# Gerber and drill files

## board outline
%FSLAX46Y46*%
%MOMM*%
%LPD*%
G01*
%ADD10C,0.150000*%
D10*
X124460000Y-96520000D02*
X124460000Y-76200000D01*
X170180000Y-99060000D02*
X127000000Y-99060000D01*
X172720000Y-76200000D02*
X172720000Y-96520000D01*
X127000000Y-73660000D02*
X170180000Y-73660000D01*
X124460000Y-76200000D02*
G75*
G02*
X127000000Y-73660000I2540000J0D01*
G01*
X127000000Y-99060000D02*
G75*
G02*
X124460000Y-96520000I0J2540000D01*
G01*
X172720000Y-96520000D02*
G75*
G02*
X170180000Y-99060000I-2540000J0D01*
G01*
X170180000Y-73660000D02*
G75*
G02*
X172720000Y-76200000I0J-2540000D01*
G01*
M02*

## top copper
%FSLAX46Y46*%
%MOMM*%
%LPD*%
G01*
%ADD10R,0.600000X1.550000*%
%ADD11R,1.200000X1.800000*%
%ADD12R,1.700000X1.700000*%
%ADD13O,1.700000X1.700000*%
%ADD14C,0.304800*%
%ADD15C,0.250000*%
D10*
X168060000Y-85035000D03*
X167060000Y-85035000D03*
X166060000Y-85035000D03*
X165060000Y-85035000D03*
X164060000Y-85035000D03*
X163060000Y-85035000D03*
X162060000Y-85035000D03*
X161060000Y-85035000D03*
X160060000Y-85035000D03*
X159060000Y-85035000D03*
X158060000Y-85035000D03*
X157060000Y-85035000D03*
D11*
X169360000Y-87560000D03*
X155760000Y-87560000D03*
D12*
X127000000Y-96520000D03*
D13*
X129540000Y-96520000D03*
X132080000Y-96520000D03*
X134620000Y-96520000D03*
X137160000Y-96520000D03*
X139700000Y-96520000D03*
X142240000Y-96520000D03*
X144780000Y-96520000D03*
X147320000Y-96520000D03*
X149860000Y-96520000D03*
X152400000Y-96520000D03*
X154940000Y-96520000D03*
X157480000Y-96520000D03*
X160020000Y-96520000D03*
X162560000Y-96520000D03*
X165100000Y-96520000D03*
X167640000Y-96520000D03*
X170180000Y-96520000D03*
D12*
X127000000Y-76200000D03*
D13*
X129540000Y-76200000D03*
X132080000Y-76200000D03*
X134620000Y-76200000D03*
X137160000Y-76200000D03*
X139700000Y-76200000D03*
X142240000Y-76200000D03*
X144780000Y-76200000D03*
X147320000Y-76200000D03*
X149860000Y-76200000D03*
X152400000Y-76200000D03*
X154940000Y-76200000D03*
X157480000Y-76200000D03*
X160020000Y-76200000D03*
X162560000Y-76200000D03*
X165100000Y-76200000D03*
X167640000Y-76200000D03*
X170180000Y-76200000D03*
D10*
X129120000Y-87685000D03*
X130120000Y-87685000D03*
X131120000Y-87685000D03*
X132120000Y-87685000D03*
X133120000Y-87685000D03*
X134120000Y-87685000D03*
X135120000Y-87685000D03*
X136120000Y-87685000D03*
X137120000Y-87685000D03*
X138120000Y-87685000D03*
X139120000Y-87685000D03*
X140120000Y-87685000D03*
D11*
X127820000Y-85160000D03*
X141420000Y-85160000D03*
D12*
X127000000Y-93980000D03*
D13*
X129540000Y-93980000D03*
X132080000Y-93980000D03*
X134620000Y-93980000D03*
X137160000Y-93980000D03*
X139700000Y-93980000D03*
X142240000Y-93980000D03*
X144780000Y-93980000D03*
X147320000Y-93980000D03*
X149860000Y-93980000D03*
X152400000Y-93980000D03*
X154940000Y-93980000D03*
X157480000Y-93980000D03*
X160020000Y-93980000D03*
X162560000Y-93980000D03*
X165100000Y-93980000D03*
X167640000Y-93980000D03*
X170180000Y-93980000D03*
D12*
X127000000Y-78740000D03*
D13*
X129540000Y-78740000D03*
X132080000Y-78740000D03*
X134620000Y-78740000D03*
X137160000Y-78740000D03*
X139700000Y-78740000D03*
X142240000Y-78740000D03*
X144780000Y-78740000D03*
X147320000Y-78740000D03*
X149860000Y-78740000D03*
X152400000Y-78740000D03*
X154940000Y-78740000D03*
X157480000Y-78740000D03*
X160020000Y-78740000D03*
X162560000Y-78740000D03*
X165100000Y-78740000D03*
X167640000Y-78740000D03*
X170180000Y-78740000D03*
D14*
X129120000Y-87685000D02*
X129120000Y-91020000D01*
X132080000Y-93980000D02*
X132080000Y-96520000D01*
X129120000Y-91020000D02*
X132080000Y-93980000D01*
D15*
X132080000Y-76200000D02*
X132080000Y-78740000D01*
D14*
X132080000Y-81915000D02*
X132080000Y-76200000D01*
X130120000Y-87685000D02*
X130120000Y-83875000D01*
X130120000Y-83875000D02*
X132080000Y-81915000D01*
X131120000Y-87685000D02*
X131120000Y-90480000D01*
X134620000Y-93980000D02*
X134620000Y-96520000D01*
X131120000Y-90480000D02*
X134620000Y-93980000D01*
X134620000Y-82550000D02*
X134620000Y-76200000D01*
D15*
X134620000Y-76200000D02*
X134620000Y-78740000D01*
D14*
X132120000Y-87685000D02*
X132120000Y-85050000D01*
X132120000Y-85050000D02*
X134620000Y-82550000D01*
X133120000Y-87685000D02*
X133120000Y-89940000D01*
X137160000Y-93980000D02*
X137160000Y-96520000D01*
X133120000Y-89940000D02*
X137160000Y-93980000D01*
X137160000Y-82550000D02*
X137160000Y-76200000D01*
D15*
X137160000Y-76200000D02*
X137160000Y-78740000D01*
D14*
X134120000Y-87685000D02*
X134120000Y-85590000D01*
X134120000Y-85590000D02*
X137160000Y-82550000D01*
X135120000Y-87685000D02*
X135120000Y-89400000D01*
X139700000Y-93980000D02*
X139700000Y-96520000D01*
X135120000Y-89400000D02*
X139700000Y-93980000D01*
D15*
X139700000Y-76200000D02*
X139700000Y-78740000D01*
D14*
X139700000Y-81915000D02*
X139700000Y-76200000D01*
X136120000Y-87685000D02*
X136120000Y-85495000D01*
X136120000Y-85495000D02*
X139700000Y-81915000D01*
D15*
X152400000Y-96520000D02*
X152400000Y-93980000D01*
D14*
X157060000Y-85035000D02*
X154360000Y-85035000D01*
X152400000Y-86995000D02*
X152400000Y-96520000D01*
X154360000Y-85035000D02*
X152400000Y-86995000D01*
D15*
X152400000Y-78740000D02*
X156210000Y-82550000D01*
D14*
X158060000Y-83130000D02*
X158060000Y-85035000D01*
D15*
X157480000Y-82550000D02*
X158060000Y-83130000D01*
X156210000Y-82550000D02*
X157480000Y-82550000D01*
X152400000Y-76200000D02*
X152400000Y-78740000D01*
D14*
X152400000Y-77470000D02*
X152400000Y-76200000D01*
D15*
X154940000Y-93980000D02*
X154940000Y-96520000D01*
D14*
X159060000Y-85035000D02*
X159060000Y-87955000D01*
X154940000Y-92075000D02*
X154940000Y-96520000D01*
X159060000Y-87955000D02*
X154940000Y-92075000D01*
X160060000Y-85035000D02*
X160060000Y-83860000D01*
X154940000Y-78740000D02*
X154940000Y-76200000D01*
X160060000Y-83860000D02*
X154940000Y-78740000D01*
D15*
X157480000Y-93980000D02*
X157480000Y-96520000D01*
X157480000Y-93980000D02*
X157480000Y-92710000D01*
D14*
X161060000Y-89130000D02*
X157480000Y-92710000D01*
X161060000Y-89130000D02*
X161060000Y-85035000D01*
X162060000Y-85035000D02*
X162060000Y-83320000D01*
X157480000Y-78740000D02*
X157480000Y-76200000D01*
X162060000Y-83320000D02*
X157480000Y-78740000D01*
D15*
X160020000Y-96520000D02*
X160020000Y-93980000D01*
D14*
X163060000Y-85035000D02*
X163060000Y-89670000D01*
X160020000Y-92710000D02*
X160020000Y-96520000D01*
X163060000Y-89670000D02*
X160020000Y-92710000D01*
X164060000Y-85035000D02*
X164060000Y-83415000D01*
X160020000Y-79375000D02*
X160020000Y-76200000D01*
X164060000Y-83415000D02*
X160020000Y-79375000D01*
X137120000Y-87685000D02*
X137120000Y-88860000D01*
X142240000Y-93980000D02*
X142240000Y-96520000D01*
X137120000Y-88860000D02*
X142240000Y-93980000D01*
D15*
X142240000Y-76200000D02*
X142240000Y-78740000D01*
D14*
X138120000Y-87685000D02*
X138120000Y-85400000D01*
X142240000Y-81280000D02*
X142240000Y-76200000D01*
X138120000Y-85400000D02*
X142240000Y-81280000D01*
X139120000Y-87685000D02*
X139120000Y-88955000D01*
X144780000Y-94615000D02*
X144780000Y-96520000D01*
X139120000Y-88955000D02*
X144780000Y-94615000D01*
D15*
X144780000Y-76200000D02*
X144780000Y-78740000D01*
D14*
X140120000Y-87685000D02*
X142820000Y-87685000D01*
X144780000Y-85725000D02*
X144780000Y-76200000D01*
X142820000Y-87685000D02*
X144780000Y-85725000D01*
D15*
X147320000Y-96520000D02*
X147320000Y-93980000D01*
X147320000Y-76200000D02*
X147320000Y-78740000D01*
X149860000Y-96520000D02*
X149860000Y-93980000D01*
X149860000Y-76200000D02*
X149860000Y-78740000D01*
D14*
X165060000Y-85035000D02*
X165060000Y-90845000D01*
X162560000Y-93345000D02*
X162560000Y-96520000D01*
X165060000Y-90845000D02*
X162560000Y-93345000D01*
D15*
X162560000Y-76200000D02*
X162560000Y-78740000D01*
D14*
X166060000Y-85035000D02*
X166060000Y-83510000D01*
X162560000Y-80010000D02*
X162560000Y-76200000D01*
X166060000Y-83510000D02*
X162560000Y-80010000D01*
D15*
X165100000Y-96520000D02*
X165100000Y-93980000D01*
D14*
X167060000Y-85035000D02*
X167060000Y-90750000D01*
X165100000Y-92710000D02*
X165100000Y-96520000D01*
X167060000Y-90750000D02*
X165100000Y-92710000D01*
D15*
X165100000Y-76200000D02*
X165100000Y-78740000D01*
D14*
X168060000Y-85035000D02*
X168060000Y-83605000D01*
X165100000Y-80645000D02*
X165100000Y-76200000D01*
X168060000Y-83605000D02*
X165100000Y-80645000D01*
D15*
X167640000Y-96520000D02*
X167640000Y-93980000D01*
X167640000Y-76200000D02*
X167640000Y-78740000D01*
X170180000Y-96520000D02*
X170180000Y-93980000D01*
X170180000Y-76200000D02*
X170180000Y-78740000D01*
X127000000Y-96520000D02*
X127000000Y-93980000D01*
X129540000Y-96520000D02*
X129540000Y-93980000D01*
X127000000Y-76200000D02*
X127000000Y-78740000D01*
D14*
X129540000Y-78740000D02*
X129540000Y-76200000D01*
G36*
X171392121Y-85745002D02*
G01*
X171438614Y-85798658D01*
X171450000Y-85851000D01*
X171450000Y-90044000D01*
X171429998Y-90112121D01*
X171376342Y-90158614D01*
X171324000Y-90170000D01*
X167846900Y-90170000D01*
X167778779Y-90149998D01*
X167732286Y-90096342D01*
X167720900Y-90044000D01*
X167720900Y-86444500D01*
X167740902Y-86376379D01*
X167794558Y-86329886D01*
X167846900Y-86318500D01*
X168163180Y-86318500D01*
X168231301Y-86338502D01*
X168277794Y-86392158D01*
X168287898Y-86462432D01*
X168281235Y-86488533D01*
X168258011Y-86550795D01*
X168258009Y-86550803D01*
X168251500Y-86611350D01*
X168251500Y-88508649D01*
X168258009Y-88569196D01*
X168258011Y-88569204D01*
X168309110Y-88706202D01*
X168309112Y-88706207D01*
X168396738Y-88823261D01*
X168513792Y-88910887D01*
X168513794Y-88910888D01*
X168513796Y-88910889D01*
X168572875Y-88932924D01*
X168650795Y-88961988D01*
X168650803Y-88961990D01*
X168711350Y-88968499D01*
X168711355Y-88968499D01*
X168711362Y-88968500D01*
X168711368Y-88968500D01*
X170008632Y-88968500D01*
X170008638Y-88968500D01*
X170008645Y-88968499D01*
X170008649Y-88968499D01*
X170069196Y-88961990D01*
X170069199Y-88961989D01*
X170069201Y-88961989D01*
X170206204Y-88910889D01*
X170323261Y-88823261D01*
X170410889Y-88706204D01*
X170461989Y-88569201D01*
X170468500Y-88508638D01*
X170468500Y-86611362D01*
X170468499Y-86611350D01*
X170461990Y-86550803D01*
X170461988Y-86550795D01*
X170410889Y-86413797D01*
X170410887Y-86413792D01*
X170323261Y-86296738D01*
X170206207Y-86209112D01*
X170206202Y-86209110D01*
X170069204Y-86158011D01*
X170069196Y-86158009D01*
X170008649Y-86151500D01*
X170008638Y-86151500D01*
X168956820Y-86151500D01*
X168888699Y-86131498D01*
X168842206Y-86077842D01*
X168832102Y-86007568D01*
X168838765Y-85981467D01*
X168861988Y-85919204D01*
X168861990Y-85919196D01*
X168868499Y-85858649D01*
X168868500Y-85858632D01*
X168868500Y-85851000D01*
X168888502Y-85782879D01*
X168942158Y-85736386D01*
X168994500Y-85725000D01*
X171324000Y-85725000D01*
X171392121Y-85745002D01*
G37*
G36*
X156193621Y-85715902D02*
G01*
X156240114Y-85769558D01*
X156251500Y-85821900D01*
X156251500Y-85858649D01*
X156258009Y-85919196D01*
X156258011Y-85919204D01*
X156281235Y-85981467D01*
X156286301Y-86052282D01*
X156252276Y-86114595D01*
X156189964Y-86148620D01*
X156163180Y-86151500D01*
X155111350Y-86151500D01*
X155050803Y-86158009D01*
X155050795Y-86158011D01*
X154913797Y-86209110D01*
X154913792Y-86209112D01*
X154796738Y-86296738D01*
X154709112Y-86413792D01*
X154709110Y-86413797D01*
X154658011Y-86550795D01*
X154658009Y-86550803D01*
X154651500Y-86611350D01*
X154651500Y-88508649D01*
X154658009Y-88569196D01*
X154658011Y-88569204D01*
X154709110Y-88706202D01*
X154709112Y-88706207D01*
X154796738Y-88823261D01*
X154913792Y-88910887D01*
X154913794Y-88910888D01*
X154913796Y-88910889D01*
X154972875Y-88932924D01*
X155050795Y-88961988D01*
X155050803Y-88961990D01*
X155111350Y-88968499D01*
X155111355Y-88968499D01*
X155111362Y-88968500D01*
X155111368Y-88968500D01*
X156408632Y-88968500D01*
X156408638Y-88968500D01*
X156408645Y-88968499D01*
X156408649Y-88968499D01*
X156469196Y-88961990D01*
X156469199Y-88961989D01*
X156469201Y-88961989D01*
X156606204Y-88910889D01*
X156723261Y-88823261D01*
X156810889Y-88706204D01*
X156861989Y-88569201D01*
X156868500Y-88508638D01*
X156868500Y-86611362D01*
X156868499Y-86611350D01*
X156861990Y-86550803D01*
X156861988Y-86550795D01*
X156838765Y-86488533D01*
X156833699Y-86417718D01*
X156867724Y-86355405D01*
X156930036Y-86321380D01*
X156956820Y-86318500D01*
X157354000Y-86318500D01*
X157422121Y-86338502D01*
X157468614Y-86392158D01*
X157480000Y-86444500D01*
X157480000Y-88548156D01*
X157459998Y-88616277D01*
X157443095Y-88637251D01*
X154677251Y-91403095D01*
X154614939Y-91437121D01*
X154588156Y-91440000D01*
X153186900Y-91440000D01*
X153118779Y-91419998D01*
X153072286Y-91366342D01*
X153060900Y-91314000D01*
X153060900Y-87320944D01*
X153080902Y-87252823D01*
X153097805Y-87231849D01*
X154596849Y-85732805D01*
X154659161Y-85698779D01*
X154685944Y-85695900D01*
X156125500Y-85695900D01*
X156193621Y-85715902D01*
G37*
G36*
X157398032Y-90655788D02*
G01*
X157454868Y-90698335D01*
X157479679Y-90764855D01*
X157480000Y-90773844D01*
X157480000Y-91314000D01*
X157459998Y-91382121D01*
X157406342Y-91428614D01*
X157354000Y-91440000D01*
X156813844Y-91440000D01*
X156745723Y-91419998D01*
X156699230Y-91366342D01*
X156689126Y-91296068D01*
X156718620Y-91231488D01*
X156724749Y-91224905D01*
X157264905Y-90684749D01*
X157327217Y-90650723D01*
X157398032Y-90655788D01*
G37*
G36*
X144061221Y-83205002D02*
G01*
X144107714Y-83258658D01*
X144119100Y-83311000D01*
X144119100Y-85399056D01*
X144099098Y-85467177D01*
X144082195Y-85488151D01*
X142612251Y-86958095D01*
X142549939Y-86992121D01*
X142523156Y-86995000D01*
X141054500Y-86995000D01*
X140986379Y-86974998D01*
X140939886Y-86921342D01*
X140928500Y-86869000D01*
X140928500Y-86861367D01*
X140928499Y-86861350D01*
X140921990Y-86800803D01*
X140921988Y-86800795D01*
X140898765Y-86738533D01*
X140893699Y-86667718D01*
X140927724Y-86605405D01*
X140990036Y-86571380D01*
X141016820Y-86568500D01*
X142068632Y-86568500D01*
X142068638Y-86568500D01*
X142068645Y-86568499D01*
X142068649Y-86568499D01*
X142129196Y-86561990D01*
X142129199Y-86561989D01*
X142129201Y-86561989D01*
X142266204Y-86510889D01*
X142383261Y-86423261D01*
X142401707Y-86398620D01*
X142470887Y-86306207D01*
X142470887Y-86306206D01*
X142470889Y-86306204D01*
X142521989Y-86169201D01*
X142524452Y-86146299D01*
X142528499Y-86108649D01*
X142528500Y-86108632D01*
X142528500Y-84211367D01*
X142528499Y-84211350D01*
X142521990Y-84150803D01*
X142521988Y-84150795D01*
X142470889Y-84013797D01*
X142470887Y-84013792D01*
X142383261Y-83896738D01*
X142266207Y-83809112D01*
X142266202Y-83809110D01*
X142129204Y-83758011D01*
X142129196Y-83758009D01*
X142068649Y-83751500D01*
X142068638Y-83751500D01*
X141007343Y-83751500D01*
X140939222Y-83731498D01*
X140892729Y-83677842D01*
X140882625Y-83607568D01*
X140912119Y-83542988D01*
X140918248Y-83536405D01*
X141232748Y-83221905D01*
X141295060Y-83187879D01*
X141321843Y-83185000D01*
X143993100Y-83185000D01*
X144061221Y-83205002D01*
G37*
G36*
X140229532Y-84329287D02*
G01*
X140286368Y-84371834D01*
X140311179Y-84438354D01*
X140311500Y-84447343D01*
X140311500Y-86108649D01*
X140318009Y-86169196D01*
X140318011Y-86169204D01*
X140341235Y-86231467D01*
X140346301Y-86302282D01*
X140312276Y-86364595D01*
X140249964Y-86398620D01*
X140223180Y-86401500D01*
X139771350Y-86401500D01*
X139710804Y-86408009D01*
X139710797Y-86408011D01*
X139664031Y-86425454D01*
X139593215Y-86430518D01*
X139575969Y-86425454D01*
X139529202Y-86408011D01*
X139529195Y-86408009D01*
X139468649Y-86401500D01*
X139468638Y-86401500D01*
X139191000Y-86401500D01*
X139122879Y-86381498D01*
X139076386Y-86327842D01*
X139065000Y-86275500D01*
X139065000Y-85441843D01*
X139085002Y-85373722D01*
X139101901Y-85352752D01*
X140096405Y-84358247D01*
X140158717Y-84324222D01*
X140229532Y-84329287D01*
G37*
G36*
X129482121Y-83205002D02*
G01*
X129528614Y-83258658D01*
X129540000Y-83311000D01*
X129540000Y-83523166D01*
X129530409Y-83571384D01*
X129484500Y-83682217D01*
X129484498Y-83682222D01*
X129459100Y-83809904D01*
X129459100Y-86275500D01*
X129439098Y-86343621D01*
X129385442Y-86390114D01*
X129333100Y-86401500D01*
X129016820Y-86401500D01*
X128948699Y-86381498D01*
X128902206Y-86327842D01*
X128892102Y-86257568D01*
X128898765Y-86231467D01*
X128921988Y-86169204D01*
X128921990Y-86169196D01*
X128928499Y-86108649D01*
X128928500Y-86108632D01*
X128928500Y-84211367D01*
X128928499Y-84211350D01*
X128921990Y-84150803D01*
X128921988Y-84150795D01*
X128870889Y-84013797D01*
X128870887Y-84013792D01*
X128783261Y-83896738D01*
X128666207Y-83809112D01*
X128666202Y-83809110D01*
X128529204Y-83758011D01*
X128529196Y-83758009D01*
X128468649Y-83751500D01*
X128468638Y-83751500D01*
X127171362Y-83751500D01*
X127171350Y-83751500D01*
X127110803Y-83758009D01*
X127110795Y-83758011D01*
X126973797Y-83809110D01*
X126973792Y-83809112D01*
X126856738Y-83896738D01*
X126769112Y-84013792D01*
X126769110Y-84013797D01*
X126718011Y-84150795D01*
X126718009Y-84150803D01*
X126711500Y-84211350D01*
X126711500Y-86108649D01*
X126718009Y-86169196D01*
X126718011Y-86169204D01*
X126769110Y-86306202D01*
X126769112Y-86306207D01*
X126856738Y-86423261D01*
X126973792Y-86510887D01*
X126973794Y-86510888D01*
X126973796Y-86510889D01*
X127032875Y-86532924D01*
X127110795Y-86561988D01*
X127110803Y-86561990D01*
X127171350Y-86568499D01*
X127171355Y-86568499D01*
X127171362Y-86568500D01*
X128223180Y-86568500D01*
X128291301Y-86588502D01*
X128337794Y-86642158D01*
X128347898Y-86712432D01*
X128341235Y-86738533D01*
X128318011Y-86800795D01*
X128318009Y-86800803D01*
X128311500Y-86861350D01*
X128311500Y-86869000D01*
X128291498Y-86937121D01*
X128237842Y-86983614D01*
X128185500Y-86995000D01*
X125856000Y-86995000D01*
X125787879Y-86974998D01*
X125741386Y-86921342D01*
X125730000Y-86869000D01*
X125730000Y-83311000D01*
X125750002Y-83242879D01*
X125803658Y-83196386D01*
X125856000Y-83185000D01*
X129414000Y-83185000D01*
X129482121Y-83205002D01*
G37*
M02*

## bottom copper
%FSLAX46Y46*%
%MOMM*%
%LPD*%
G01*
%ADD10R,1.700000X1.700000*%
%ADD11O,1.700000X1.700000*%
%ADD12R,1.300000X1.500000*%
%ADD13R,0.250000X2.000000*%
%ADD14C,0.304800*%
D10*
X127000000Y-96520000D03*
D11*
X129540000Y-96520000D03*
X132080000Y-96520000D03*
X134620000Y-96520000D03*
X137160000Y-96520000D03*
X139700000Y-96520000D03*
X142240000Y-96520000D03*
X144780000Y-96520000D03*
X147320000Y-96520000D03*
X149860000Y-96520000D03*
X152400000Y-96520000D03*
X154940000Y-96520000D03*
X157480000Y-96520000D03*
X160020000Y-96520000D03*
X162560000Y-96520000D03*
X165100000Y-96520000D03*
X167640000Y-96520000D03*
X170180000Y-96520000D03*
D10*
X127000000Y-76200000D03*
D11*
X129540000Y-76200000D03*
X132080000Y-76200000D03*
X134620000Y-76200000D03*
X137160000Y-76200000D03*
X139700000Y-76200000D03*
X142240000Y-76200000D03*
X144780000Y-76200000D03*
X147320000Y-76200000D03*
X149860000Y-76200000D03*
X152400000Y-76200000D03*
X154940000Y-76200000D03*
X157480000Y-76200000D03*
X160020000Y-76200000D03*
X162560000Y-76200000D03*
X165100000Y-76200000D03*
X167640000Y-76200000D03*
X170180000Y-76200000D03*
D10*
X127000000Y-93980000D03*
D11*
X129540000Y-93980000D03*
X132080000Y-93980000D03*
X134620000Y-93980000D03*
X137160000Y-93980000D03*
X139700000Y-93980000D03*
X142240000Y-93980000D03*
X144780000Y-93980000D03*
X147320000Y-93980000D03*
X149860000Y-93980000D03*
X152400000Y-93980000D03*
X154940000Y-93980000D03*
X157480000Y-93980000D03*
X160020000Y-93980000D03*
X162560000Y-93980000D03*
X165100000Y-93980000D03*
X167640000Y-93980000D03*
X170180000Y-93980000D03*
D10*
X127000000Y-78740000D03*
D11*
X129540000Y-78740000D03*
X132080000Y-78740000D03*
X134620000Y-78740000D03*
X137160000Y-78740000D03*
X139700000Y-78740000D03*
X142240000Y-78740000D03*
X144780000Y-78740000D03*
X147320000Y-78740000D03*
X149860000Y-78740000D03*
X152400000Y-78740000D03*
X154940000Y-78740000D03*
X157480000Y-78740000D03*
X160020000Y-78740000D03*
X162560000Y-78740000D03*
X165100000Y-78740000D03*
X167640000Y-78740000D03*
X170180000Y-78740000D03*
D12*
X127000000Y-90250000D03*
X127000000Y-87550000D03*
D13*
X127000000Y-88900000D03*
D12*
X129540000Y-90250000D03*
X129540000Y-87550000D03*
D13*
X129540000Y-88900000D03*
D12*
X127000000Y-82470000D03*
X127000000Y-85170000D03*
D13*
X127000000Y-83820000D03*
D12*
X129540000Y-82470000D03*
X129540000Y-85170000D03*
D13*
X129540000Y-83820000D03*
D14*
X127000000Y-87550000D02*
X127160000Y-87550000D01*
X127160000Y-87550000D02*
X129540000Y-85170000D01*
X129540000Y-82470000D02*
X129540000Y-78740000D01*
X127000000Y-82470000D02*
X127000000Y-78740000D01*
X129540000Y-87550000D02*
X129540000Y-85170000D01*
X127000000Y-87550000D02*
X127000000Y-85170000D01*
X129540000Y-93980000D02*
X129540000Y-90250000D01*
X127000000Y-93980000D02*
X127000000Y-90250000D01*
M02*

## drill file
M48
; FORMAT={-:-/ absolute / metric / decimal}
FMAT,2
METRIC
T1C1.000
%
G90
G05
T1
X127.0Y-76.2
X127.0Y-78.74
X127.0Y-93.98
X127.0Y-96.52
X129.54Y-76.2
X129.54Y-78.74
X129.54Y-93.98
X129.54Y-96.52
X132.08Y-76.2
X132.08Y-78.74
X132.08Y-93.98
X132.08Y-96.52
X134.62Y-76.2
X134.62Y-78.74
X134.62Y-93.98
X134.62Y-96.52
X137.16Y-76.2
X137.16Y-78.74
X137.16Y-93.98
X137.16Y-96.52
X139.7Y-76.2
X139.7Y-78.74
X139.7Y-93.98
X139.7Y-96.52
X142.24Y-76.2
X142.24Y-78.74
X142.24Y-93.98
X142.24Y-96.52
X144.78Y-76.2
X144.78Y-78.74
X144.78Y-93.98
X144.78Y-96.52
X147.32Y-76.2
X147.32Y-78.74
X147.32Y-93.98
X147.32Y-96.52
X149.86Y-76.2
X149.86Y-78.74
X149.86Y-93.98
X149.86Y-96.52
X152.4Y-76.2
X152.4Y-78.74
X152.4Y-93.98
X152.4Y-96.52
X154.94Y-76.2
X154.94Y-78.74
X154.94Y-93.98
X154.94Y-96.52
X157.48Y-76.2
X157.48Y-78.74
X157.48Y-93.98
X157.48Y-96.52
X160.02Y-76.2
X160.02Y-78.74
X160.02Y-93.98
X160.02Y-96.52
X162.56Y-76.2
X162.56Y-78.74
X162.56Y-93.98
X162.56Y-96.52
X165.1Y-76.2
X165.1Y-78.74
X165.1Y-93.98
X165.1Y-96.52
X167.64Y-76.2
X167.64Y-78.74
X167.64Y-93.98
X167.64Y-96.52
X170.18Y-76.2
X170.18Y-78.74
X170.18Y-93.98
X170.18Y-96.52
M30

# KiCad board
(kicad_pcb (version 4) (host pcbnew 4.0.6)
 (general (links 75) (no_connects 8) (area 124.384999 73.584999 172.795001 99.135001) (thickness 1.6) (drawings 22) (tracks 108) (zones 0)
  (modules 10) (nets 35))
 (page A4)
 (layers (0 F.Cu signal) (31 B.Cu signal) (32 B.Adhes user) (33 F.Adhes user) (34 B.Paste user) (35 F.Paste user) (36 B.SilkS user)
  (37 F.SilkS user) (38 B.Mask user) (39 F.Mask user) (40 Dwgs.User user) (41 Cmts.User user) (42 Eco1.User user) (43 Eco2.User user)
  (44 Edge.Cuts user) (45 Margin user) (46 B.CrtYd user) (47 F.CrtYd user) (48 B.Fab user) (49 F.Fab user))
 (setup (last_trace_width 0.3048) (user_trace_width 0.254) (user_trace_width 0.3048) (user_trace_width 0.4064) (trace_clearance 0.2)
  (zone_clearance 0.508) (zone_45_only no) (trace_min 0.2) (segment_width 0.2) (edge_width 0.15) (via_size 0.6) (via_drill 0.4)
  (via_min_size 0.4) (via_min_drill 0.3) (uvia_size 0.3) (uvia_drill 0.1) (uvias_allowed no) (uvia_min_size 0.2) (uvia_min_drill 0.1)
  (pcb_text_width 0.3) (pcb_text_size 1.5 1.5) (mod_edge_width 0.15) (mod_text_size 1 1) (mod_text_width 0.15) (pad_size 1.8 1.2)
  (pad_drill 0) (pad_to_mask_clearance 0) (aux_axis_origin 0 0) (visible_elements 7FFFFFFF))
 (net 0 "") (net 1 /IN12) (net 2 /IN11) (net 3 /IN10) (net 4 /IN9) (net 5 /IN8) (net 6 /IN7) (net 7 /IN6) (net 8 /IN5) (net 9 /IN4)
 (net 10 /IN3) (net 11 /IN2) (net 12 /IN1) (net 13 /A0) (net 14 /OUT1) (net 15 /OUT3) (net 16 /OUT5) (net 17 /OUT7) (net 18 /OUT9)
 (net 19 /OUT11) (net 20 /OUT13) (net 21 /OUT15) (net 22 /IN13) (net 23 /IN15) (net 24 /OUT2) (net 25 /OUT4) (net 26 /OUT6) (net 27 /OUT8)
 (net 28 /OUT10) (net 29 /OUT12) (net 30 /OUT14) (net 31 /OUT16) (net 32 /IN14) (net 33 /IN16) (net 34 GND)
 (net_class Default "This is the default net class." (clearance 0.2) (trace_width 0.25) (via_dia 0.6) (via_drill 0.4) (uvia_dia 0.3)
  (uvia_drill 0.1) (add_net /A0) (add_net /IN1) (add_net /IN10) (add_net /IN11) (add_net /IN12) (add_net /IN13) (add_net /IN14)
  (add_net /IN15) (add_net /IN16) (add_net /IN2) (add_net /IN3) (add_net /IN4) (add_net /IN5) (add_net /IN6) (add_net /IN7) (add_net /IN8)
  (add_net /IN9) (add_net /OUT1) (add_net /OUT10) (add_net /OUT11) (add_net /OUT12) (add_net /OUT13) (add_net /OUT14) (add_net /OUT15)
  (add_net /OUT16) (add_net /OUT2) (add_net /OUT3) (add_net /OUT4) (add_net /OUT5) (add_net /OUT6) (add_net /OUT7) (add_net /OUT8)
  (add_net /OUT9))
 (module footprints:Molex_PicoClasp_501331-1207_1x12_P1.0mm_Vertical (layer F.Cu) (at 162.56 86.36 270)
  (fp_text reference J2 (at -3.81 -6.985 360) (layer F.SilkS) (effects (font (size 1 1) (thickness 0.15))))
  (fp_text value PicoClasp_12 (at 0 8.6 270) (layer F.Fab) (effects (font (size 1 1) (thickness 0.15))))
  (pad 1 smd rect (at -1.325 -5.5 270) (size 1.55 0.6) (layers F.Cu F.Paste F.Mask) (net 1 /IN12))
  (pad 2 smd rect (at -1.325 -4.5 270) (size 1.55 0.6) (layers F.Cu F.Paste F.Mask) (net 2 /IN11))
  (pad 3 smd rect (at -1.325 -3.5 270) (size 1.55 0.6) (layers F.Cu F.Paste F.Mask) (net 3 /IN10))
  (pad 4 smd rect (at -1.325 -2.5 270) (size 1.55 0.6) (layers F.Cu F.Paste F.Mask) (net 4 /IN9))
  (pad 5 smd rect (at -1.325 -1.5 270) (size 1.55 0.6) (layers F.Cu F.Paste F.Mask) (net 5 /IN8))
  (pad 6 smd rect (at -1.325 -0.5 270) (size 1.55 0.6) (layers F.Cu F.Paste F.Mask) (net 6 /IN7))
  (pad 7 smd rect (at -1.325 0.5 270) (size 1.55 0.6) (layers F.Cu F.Paste F.Mask) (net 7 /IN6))
  (pad 8 smd rect (at -1.325 1.5 270) (size 1.55 0.6) (layers F.Cu F.Paste F.Mask) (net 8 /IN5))
  (pad 9 smd rect (at -1.325 2.5 270) (size 1.55 0.6) (layers F.Cu F.Paste F.Mask) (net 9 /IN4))
  (pad 10 smd rect (at -1.325 3.5 270) (size 1.55 0.6) (layers F.Cu F.Paste F.Mask) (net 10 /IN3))
  (pad 11 smd rect (at -1.325 4.5 270) (size 1.55 0.6) (layers F.Cu F.Paste F.Mask) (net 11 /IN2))
  (pad 12 smd rect (at -1.325 5.5 270) (size 1.55 0.6) (layers F.Cu F.Paste F.Mask) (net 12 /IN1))
  (pad 13 smd rect (at 1.2 -6.8 270) (size 1.8 1.2) (layers F.Cu F.Paste F.Mask))
  (pad 13 smd rect (at 1.2 6.8 270) (size 1.8 1.2) (layers F.Cu F.Paste F.Mask)))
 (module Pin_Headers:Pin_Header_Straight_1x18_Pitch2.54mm (layer F.Cu) (at 127 96.52 90)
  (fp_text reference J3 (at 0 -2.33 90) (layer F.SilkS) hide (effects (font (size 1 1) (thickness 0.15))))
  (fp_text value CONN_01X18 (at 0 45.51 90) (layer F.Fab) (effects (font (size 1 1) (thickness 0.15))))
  (pad 1 thru_hole rect (at 0 0 90) (size 1.7 1.7) (drill 1) (layers *.Cu *.Mask) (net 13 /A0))
  (pad 2 thru_hole oval (at 0 2.54 90) (size 1.7 1.7) (drill 1) (layers *.Cu *.Mask) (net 13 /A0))
  (pad 3 thru_hole oval (at 0 5.08 90) (size 1.7 1.7) (drill 1) (layers *.Cu *.Mask) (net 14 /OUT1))
  (pad 4 thru_hole oval (at 0 7.62 90) (size 1.7 1.7) (drill 1) (layers *.Cu *.Mask) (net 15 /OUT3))
  (pad 5 thru_hole oval (at 0 10.16 90) (size 1.7 1.7) (drill 1) (layers *.Cu *.Mask) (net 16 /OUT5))
  (pad 6 thru_hole oval (at 0 12.7 90) (size 1.7 1.7) (drill 1) (layers *.Cu *.Mask) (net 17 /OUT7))
  (pad 7 thru_hole oval (at 0 15.24 90) (size 1.7 1.7) (drill 1) (layers *.Cu *.Mask) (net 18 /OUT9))
  (pad 8 thru_hole oval (at 0 17.78 90) (size 1.7 1.7) (drill 1) (layers *.Cu *.Mask) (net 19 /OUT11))
  (pad 9 thru_hole oval (at 0 20.32 90) (size 1.7 1.7) (drill 1) (layers *.Cu *.Mask) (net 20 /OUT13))
  (pad 10 thru_hole oval (at 0 22.86 90) (size 1.7 1.7) (drill 1) (layers *.Cu *.Mask) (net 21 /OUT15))
  (pad 11 thru_hole oval (at 0 25.4 90) (size 1.7 1.7) (drill 1) (layers *.Cu *.Mask) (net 12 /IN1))
  (pad 12 thru_hole oval (at 0 27.94 90) (size 1.7 1.7) (drill 1) (layers *.Cu *.Mask) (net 10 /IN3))
  (pad 13 thru_hole oval (at 0 30.48 90) (size 1.7 1.7) (drill 1) (layers *.Cu *.Mask) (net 8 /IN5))
  (pad 14 thru_hole oval (at 0 33.02 90) (size 1.7 1.7) (drill 1) (layers *.Cu *.Mask) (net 6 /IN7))
  (pad 15 thru_hole oval (at 0 35.56 90) (size 1.7 1.7) (drill 1) (layers *.Cu *.Mask) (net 4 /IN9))
  (pad 16 thru_hole oval (at 0 38.1 90) (size 1.7 1.7) (drill 1) (layers *.Cu *.Mask) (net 2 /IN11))
  (pad 17 thru_hole oval (at 0 40.64 90) (size 1.7 1.7) (drill 1) (layers *.Cu *.Mask) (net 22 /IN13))
  (pad 18 thru_hole oval (at 0 43.18 90) (size 1.7 1.7) (drill 1) (layers *.Cu *.Mask) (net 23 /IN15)))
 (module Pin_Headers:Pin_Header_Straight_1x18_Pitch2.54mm (layer F.Cu) (at 127 76.2 90)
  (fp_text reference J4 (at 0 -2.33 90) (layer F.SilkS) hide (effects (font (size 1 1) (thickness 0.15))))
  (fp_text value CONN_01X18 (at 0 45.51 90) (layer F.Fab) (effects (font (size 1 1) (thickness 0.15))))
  (pad 1 thru_hole rect (at 0 0 90) (size 1.7 1.7) (drill 1) (layers *.Cu *.Mask) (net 13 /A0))
  (pad 2 thru_hole oval (at 0 2.54 90) (size 1.7 1.7) (drill 1) (layers *.Cu *.Mask) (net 13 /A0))
  (pad 3 thru_hole oval (at 0 5.08 90) (size 1.7 1.7) (drill 1) (layers *.Cu *.Mask) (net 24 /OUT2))
  (pad 4 thru_hole oval (at 0 7.62 90) (size 1.7 1.7) (drill 1) (layers *.Cu *.Mask) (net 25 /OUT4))
  (pad 5 thru_hole oval (at 0 10.16 90) (size 1.7 1.7) (drill 1) (layers *.Cu *.Mask) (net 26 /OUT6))
  (pad 6 thru_hole oval (at 0 12.7 90) (size 1.7 1.7) (drill 1) (layers *.Cu *.Mask) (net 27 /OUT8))
  (pad 7 thru_hole oval (at 0 15.24 90) (size 1.7 1.7) (drill 1) (layers *.Cu *.Mask) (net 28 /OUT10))
  (pad 8 thru_hole oval (at 0 17.78 90) (size 1.7 1.7) (drill 1) (layers *.Cu *.Mask) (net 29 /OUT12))
  (pad 9 thru_hole oval (at 0 20.32 90) (size 1.7 1.7) (drill 1) (layers *.Cu *.Mask) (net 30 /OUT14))
  (pad 10 thru_hole oval (at 0 22.86 90) (size 1.7 1.7) (drill 1) (layers *.Cu *.Mask) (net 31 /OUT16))
  (pad 11 thru_hole oval (at 0 25.4 90) (size 1.7 1.7) (drill 1) (layers *.Cu *.Mask) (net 11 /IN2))
  (pad 12 thru_hole oval (at 0 27.94 90) (size 1.7 1.7) (drill 1) (layers *.Cu *.Mask) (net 9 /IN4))
  (pad 13 thru_hole oval (at 0 30.48 90) (size 1.7 1.7) (drill 1) (layers *.Cu *.Mask) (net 7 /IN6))
  (pad 14 thru_hole oval (at 0 33.02 90) (size 1.7 1.7) (drill 1) (layers *.Cu *.Mask) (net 5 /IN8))
  (pad 15 thru_hole oval (at 0 35.56 90) (size 1.7 1.7) (drill 1) (layers *.Cu *.Mask) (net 3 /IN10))
  (pad 16 thru_hole oval (at 0 38.1 90) (size 1.7 1.7) (drill 1) (layers *.Cu *.Mask) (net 1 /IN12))
  (pad 17 thru_hole oval (at 0 40.64 90) (size 1.7 1.7) (drill 1) (layers *.Cu *.Mask) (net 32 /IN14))
  (pad 18 thru_hole oval (at 0 43.18 90) (size 1.7 1.7) (drill 1) (layers *.Cu *.Mask) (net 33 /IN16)))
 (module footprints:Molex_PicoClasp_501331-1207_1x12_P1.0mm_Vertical (layer F.Cu) (at 134.62 86.36 90)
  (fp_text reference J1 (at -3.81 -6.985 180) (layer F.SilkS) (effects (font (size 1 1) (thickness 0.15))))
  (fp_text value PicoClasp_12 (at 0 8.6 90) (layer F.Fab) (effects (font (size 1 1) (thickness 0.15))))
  (pad 1 smd rect (at -1.325 -5.5 90) (size 1.55 0.6) (layers F.Cu F.Paste F.Mask) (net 14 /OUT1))
  (pad 2 smd rect (at -1.325 -4.5 90) (size 1.55 0.6) (layers F.Cu F.Paste F.Mask) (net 24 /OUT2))
  (pad 3 smd rect (at -1.325 -3.5 90) (size 1.55 0.6) (layers F.Cu F.Paste F.Mask) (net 15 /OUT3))
  (pad 4 smd rect (at -1.325 -2.5 90) (size 1.55 0.6) (layers F.Cu F.Paste F.Mask) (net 25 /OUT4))
  (pad 5 smd rect (at -1.325 -1.5 90) (size 1.55 0.6) (layers F.Cu F.Paste F.Mask) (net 16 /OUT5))
  (pad 6 smd rect (at -1.325 -0.5 90) (size 1.55 0.6) (layers F.Cu F.Paste F.Mask) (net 26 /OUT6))
  (pad 7 smd rect (at -1.325 0.5 90) (size 1.55 0.6) (layers F.Cu F.Paste F.Mask) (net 17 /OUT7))
  (pad 8 smd rect (at -1.325 1.5 90) (size 1.55 0.6) (layers F.Cu F.Paste F.Mask) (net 27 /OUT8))
  (pad 9 smd rect (at -1.325 2.5 90) (size 1.55 0.6) (layers F.Cu F.Paste F.Mask) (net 18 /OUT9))
  (pad 10 smd rect (at -1.325 3.5 90) (size 1.55 0.6) (layers F.Cu F.Paste F.Mask) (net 28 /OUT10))
  (pad 11 smd rect (at -1.325 4.5 90) (size 1.55 0.6) (layers F.Cu F.Paste F.Mask) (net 19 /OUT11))
  (pad 12 smd rect (at -1.325 5.5 90) (size 1.55 0.6) (layers F.Cu F.Paste F.Mask) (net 29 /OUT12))
  (pad 13 smd rect (at 1.2 -6.8 90) (size 1.8 1.2) (layers F.Cu F.Paste F.Mask))
  (pad 13 smd rect (at 1.2 6.8 90) (size 1.8 1.2) (layers F.Cu F.Paste F.Mask)))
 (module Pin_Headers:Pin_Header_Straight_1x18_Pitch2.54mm (layer F.Cu) (at 127 93.98 90)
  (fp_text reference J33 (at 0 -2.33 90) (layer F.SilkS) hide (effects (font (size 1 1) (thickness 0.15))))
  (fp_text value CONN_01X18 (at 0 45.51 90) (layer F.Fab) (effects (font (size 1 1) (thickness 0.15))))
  (pad 1 thru_hole rect (at 0 0 90) (size 1.7 1.7) (drill 1) (layers *.Cu *.Mask) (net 13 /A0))
  (pad 2 thru_hole oval (at 0 2.54 90) (size 1.7 1.7) (drill 1) (layers *.Cu *.Mask) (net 13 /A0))
  (pad 3 thru_hole oval (at 0 5.08 90) (size 1.7 1.7) (drill 1) (layers *.Cu *.Mask) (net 14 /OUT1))
  (pad 4 thru_hole oval (at 0 7.62 90) (size 1.7 1.7) (drill 1) (layers *.Cu *.Mask) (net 15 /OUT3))
  (pad 5 thru_hole oval (at 0 10.16 90) (size 1.7 1.7) (drill 1) (layers *.Cu *.Mask) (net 16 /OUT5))
  (pad 6 thru_hole oval (at 0 12.7 90) (size 1.7 1.7) (drill 1) (layers *.Cu *.Mask) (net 17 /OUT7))
  (pad 7 thru_hole oval (at 0 15.24 90) (size 1.7 1.7) (drill 1) (layers *.Cu *.Mask) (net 18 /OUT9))
  (pad 8 thru_hole oval (at 0 17.78 90) (size 1.7 1.7) (drill 1) (layers *.Cu *.Mask) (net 19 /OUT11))
  (pad 9 thru_hole oval (at 0 20.32 90) (size 1.7 1.7) (drill 1) (layers *.Cu *.Mask) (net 20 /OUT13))
  (pad 10 thru_hole oval (at 0 22.86 90) (size 1.7 1.7) (drill 1) (layers *.Cu *.Mask) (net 21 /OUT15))
  (pad 11 thru_hole oval (at 0 25.4 90) (size 1.7 1.7) (drill 1) (layers *.Cu *.Mask) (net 12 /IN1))
  (pad 12 thru_hole oval (at 0 27.94 90) (size 1.7 1.7) (drill 1) (layers *.Cu *.Mask) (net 10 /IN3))
  (pad 13 thru_hole oval (at 0 30.48 90) (size 1.7 1.7) (drill 1) (layers *.Cu *.Mask) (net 8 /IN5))
  (pad 14 thru_hole oval (at 0 33.02 90) (size 1.7 1.7) (drill 1) (layers *.Cu *.Mask) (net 6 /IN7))
  (pad 15 thru_hole oval (at 0 35.56 90) (size 1.7 1.7) (drill 1) (layers *.Cu *.Mask) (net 4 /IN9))
  (pad 16 thru_hole oval (at 0 38.1 90) (size 1.7 1.7) (drill 1) (layers *.Cu *.Mask) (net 2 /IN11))
  (pad 17 thru_hole oval (at 0 40.64 90) (size 1.7 1.7) (drill 1) (layers *.Cu *.Mask) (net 22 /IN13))
  (pad 18 thru_hole oval (at 0 43.18 90) (size 1.7 1.7) (drill 1) (layers *.Cu *.Mask) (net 23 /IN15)))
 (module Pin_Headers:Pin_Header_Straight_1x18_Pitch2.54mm (layer F.Cu) (at 127 78.74 90)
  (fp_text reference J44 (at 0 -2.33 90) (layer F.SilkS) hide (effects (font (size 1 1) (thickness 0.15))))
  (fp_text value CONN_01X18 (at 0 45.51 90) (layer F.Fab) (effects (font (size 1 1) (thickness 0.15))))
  (pad 1 thru_hole rect (at 0 0 90) (size 1.7 1.7) (drill 1) (layers *.Cu *.Mask) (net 13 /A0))
  (pad 2 thru_hole oval (at 0 2.54 90) (size 1.7 1.7) (drill 1) (layers *.Cu *.Mask) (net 13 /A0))
  (pad 3 thru_hole oval (at 0 5.08 90) (size 1.7 1.7) (drill 1) (layers *.Cu *.Mask) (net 24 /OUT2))
  (pad 4 thru_hole oval (at 0 7.62 90) (size 1.7 1.7) (drill 1) (layers *.Cu *.Mask) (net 25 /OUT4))
  (pad 5 thru_hole oval (at 0 10.16 90) (size 1.7 1.7) (drill 1) (layers *.Cu *.Mask) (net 26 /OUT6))
  (pad 6 thru_hole oval (at 0 12.7 90) (size 1.7 1.7) (drill 1) (layers *.Cu *.Mask) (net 27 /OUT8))
  (pad 7 thru_hole oval (at 0 15.24 90) (size 1.7 1.7) (drill 1) (layers *.Cu *.Mask) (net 28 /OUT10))
  (pad 8 thru_hole oval (at 0 17.78 90) (size 1.7 1.7) (drill 1) (layers *.Cu *.Mask) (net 29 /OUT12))
  (pad 9 thru_hole oval (at 0 20.32 90) (size 1.7 1.7) (drill 1) (layers *.Cu *.Mask) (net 30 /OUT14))
  (pad 10 thru_hole oval (at 0 22.86 90) (size 1.7 1.7) (drill 1) (layers *.Cu *.Mask) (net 31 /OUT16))
  (pad 11 thru_hole oval (at 0 25.4 90) (size 1.7 1.7) (drill 1) (layers *.Cu *.Mask) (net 11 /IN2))
  (pad 12 thru_hole oval (at 0 27.94 90) (size 1.7 1.7) (drill 1) (layers *.Cu *.Mask) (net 9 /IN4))
  (pad 13 thru_hole oval (at 0 30.48 90) (size 1.7 1.7) (drill 1) (layers *.Cu *.Mask) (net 7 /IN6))
  (pad 14 thru_hole oval (at 0 33.02 90) (size 1.7 1.7) (drill 1) (layers *.Cu *.Mask) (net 5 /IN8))
  (pad 15 thru_hole oval (at 0 35.56 90) (size 1.7 1.7) (drill 1) (layers *.Cu *.Mask) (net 3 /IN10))
  (pad 16 thru_hole oval (at 0 38.1 90) (size 1.7 1.7) (drill 1) (layers *.Cu *.Mask) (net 1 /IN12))
  (pad 17 thru_hole oval (at 0 40.64 90) (size 1.7 1.7) (drill 1) (layers *.Cu *.Mask) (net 32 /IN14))
  (pad 18 thru_hole oval (at 0 43.18 90) (size 1.7 1.7) (drill 1) (layers *.Cu *.Mask) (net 33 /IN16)))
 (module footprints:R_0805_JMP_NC (layer B.Cu) (at 127 88.9 90)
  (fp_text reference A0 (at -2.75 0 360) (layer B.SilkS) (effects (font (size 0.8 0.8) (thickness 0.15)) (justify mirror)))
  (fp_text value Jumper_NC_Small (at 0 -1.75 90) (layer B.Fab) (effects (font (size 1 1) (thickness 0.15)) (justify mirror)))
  (pad 1 smd rect (at -1.35 0 90) (size 1.5 1.3) (layers B.Cu B.Paste B.Mask) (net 13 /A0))
  (pad 2 smd rect (at 1.35 0 90) (size 1.5 1.3) (layers B.Cu B.Paste B.Mask) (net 13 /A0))
  (pad 1 smd rect (at 0 0 90) (size 2 0.25) (layers B.Cu B.Paste B.Mask) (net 13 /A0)))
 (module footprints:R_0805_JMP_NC (layer B.Cu) (at 129.54 88.9 90)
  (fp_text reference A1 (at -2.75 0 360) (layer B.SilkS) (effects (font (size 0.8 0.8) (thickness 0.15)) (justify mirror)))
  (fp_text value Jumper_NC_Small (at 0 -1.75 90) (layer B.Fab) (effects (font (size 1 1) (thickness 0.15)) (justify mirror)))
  (pad 1 smd rect (at -1.35 0 90) (size 1.5 1.3) (layers B.Cu B.Paste B.Mask) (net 13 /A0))
  (pad 2 smd rect (at 1.35 0 90) (size 1.5 1.3) (layers B.Cu B.Paste B.Mask) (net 13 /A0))
  (pad 1 smd rect (at 0 0 90) (size 2 0.25) (layers B.Cu B.Paste B.Mask) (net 13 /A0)))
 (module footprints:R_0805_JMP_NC (layer B.Cu) (at 127 83.82 270)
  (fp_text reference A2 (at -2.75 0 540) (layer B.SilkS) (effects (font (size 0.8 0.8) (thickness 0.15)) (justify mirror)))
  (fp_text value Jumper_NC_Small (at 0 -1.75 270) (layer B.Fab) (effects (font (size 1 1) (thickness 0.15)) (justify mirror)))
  (pad 1 smd rect (at -1.35 0 270) (size 1.5 1.3) (layers B.Cu B.Paste B.Mask) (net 13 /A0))
  (pad 2 smd rect (at 1.35 0 270) (size 1.5 1.3) (layers B.Cu B.Paste B.Mask) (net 13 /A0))
  (pad 1 smd rect (at 0 0 270) (size 2 0.25) (layers B.Cu B.Paste B.Mask) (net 13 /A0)))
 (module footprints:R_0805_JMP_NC (layer B.Cu) (at 129.54 83.82 270)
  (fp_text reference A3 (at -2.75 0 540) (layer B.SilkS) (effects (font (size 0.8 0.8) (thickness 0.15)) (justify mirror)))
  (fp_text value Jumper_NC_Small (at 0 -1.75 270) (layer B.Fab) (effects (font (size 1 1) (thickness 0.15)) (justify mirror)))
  (pad 1 smd rect (at -1.35 0 270) (size 1.5 1.3) (layers B.Cu B.Paste B.Mask) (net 13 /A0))
  (pad 2 smd rect (at 1.35 0 270) (size 1.5 1.3) (layers B.Cu B.Paste B.Mask) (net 13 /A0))
  (pad 1 smd rect (at 0 0 270) (size 2 0.25) (layers B.Cu B.Paste B.Mask) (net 13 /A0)))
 (gr_line (start 124.46 96.52) (end 124.46 76.2) (angle 90) (layer Edge.Cuts) (width 0.15))
 (gr_line (start 170.18 99.06) (end 127 99.06) (angle 90) (layer Edge.Cuts) (width 0.15))
 (gr_line (start 172.72 76.2) (end 172.72 96.52) (angle 90) (layer Edge.Cuts) (width 0.15))
 (gr_line (start 127 73.66) (end 170.18 73.66) (angle 90) (layer Edge.Cuts) (width 0.15))
 (gr_arc (start 127 76.2) (end 124.46 76.2) (angle 90) (layer Edge.Cuts) (width 0.15))
 (gr_arc (start 127 96.52) (end 127 99.06) (angle 90) (layer Edge.Cuts) (width 0.15))
 (gr_arc (start 170.18 96.52) (end 172.72 96.52) (angle 90) (layer Edge.Cuts) (width 0.15))
 (gr_arc (start 170.18 76.2) (end 170.18 73.66) (angle 90) (layer Edge.Cuts) (width 0.15))
 (segment (start 129.12 87.685) (end 129.12 91.02) (width 0.3048) (layer F.Cu) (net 14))
 (segment (start 132.08 93.98) (end 132.08 96.52) (width 0.3048) (layer F.Cu) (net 14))
 (segment (start 129.12 91.02) (end 132.08 93.98) (width 0.3048) (layer F.Cu) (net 14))
 (segment (start 132.08 76.2) (end 132.08 78.74) (width 0.25) (layer F.Cu) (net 24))
 (segment (start 132.08 81.915) (end 132.08 76.2) (width 0.3048) (layer F.Cu) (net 24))
 (segment (start 130.12 87.685) (end 130.12 83.875) (width 0.3048) (layer F.Cu) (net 24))
 (segment (start 130.12 83.875) (end 132.08 81.915) (width 0.3048) (layer F.Cu) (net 24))
 (segment (start 131.12 87.685) (end 131.12 90.48) (width 0.3048) (layer F.Cu) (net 15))
 (segment (start 134.62 93.98) (end 134.62 96.52) (width 0.3048) (layer F.Cu) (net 15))
 (segment (start 131.12 90.48) (end 134.62 93.98) (width 0.3048) (layer F.Cu) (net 15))
 (segment (start 134.62 82.55) (end 134.62 76.2) (width 0.3048) (layer F.Cu) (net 25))
 (segment (start 134.62 76.2) (end 134.62 78.74) (width 0.25) (layer F.Cu) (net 25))
 (segment (start 132.12 87.685) (end 132.12 85.05) (width 0.3048) (layer F.Cu) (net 25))
 (segment (start 132.12 85.05) (end 134.62 82.55) (width 0.3048) (layer F.Cu) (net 25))
 (segment (start 133.12 87.685) (end 133.12 89.94) (width 0.3048) (layer F.Cu) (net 16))
 (segment (start 137.16 93.98) (end 137.16 96.52) (width 0.3048) (layer F.Cu) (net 16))
 (segment (start 133.12 89.94) (end 137.16 93.98) (width 0.3048) (layer F.Cu) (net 16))
 (segment (start 137.16 82.55) (end 137.16 76.2) (width 0.3048) (layer F.Cu) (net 26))
 (segment (start 137.16 76.2) (end 137.16 78.74) (width 0.25) (layer F.Cu) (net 26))
 (segment (start 134.12 87.685) (end 134.12 85.59) (width 0.3048) (layer F.Cu) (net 26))
 (segment (start 134.12 85.59) (end 137.16 82.55) (width 0.3048) (layer F.Cu) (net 26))
 (segment (start 135.12 87.685) (end 135.12 89.4) (width 0.3048) (layer F.Cu) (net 17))
 (segment (start 139.7 93.98) (end 139.7 96.52) (width 0.3048) (layer F.Cu) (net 17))
 (segment (start 135.12 89.4) (end 139.7 93.98) (width 0.3048) (layer F.Cu) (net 17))
 (segment (start 139.7 76.2) (end 139.7 78.74) (width 0.25) (layer F.Cu) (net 27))
 (segment (start 139.7 81.915) (end 139.7 76.2) (width 0.3048) (layer F.Cu) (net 27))
 (segment (start 136.12 87.685) (end 136.12 85.495) (width 0.3048) (layer F.Cu) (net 27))
 (segment (start 136.12 85.495) (end 139.7 81.915) (width 0.3048) (layer F.Cu) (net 27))
 (segment (start 152.4 96.52) (end 152.4 93.98) (width 0.25) (layer F.Cu) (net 12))
 (segment (start 157.06 85.035) (end 154.36 85.035) (width 0.3048) (layer F.Cu) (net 12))
 (segment (start 152.4 86.995) (end 152.4 96.52) (width 0.3048) (layer F.Cu) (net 12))
 (segment (start 154.36 85.035) (end 152.4 86.995) (width 0.3048) (layer F.Cu) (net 12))
 (segment (start 152.4 78.74) (end 156.21 82.55) (width 0.25) (layer F.Cu) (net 11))
 (segment (start 158.06 83.13) (end 158.06 85.035) (width 0.3048) (layer F.Cu) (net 11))
 (segment (start 157.48 82.55) (end 158.06 83.13) (width 0.25) (layer F.Cu) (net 11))
 (segment (start 156.21 82.55) (end 157.48 82.55) (width 0.25) (layer F.Cu) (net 11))
 (segment (start 152.4 76.2) (end 152.4 78.74) (width 0.25) (layer F.Cu) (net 11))
 (segment (start 152.4 77.47) (end 152.4 76.2) (width 0.3048) (layer F.Cu) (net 11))
 (segment (start 154.94 93.98) (end 154.94 96.52) (width 0.25) (layer F.Cu) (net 10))
 (segment (start 159.06 85.035) (end 159.06 87.955) (width 0.3048) (layer F.Cu) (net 10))
 (segment (start 154.94 92.075) (end 154.94 96.52) (width 0.3048) (layer F.Cu) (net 10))
 (segment (start 159.06 87.955) (end 154.94 92.075) (width 0.3048) (layer F.Cu) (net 10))
 (segment (start 160.06 85.035) (end 160.06 83.86) (width 0.3048) (layer F.Cu) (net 9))
 (segment (start 154.94 78.74) (end 154.94 76.2) (width 0.3048) (layer F.Cu) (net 9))
 (segment (start 160.06 83.86) (end 154.94 78.74) (width 0.3048) (layer F.Cu) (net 9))
 (segment (start 157.48 93.98) (end 157.48 96.52) (width 0.25) (layer F.Cu) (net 8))
 (segment (start 157.48 93.98) (end 157.48 92.71) (width 0.25) (layer F.Cu) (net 8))
 (segment (start 161.06 89.13) (end 157.48 92.71) (width 0.3048) (layer F.Cu) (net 8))
 (segment (start 161.06 89.13) (end 161.06 85.035) (width 0.3048) (layer F.Cu) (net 8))
 (segment (start 162.06 85.035) (end 162.06 83.32) (width 0.3048) (layer F.Cu) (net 7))
 (segment (start 157.48 78.74) (end 157.48 76.2) (width 0.3048) (layer F.Cu) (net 7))
 (segment (start 162.06 83.32) (end 157.48 78.74) (width 0.3048) (layer F.Cu) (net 7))
 (segment (start 160.02 96.52) (end 160.02 93.98) (width 0.25) (layer F.Cu) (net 6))
 (segment (start 163.06 85.035) (end 163.06 89.67) (width 0.3048) (layer F.Cu) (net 6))
 (segment (start 160.02 92.71) (end 160.02 96.52) (width 0.3048) (layer F.Cu) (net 6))
 (segment (start 163.06 89.67) (end 160.02 92.71) (width 0.3048) (layer F.Cu) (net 6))
 (segment (start 164.06 85.035) (end 164.06 83.415) (width 0.3048) (layer F.Cu) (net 5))
 (segment (start 160.02 79.375) (end 160.02 76.2) (width 0.3048) (layer F.Cu) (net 5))
 (segment (start 164.06 83.415) (end 160.02 79.375) (width 0.3048) (layer F.Cu) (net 5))
 (segment (start 137.12 87.685) (end 137.12 88.86) (width 0.3048) (layer F.Cu) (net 18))
 (segment (start 142.24 93.98) (end 142.24 96.52) (width 0.3048) (layer F.Cu) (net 18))
 (segment (start 137.12 88.86) (end 142.24 93.98) (width 0.3048) (layer F.Cu) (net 18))
 (segment (start 142.24 76.2) (end 142.24 78.74) (width 0.25) (layer F.Cu) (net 28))
 (segment (start 138.12 87.685) (end 138.12 85.4) (width 0.3048) (layer F.Cu) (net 28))
 (segment (start 142.24 81.28) (end 142.24 76.2) (width 0.3048) (layer F.Cu) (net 28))
 (segment (start 138.12 85.4) (end 142.24 81.28) (width 0.3048) (layer F.Cu) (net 28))
 (segment (start 139.12 87.685) (end 139.12 88.955) (width 0.3048) (layer F.Cu) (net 19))
 (segment (start 144.78 94.615) (end 144.78 96.52) (width 0.3048) (layer F.Cu) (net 19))
 (segment (start 139.12 88.955) (end 144.78 94.615) (width 0.3048) (layer F.Cu) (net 19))
 (segment (start 144.78 76.2) (end 144.78 78.74) (width 0.25) (layer F.Cu) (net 29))
 (segment (start 140.12 87.685) (end 142.82 87.685) (width 0.3048) (layer F.Cu) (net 29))
 (segment (start 144.78 85.725) (end 144.78 76.2) (width 0.3048) (layer F.Cu) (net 29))
 (segment (start 142.82 87.685) (end 144.78 85.725) (width 0.3048) (layer F.Cu) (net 29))
 (segment (start 147.32 96.52) (end 147.32 93.98) (width 0.25) (layer F.Cu) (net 20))
 (segment (start 147.32 76.2) (end 147.32 78.74) (width 0.25) (layer F.Cu) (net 30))
 (segment (start 149.86 96.52) (end 149.86 93.98) (width 0.25) (layer F.Cu) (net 21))
 (segment (start 149.86 76.2) (end 149.86 78.74) (width 0.25) (layer F.Cu) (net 31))
 (segment (start 165.06 85.035) (end 165.06 90.845) (width 0.3048) (layer F.Cu) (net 4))
 (segment (start 162.56 93.345) (end 162.56 96.52) (width 0.3048) (layer F.Cu) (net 4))
 (segment (start 165.06 90.845) (end 162.56 93.345) (width 0.3048) (layer F.Cu) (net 4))
 (segment (start 162.56 76.2) (end 162.56 78.74) (width 0.25) (layer F.Cu) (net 3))
 (segment (start 166.06 85.035) (end 166.06 83.51) (width 0.3048) (layer F.Cu) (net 3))
 (segment (start 162.56 80.01) (end 162.56 76.2) (width 0.3048) (layer F.Cu) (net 3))
 (segment (start 166.06 83.51) (end 162.56 80.01) (width 0.3048) (layer F.Cu) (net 3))
 (segment (start 165.1 96.52) (end 165.1 93.98) (width 0.25) (layer F.Cu) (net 2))
 (segment (start 167.06 85.035) (end 167.06 90.75) (width 0.3048) (layer F.Cu) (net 2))
 (segment (start 165.1 92.71) (end 165.1 96.52) (width 0.3048) (layer F.Cu) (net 2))
 (segment (start 167.06 90.75) (end 165.1 92.71) (width 0.3048) (layer F.Cu) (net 2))
 (segment (start 165.1 76.2) (end 165.1 78.74) (width 0.25) (layer F.Cu) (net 1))
 (segment (start 168.06 85.035) (end 168.06 83.605) (width 0.3048) (layer F.Cu) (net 1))
 (segment (start 165.1 80.645) (end 165.1 76.2) (width 0.3048) (layer F.Cu) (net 1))
 (segment (start 168.06 83.605) (end 165.1 80.645) (width 0.3048) (layer F.Cu) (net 1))
 (segment (start 167.64 96.52) (end 167.64 93.98) (width 0.25) (layer F.Cu) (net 22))
 (segment (start 167.64 76.2) (end 167.64 78.74) (width 0.25) (layer F.Cu) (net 32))
 (segment (start 170.18 96.52) (end 170.18 93.98) (width 0.25) (layer F.Cu) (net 23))
 (segment (start 170.18 76.2) (end 170.18 78.74) (width 0.25) (layer F.Cu) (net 33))
 (segment (start 127 87.55) (end 127.16 87.55) (width 0.3048) (layer B.Cu) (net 13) (status C00000))
 (segment (start 127.16 87.55) (end 129.54 85.17) (width 0.3048) (layer B.Cu) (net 13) (status C00000))
 (segment (start 129.54 82.47) (end 129.54 78.74) (width 0.3048) (layer B.Cu) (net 13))
 (segment (start 127 82.47) (end 127 78.74) (width 0.3048) (layer B.Cu) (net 13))
 (segment (start 129.54 87.55) (end 129.54 85.17) (width 0.3048) (layer B.Cu) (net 13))
 (segment (start 127 87.55) (end 127 85.17) (width 0.3048) (layer B.Cu) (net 13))
 (segment (start 129.54 93.98) (end 129.54 90.25) (width 0.3048) (layer B.Cu) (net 13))
 (segment (start 127 93.98) (end 127 90.25) (width 0.3048) (layer B.Cu) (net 13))
 (segment (start 127 96.52) (end 127 93.98) (width 0.25) (layer F.Cu) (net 13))
 (segment (start 129.54 96.52) (end 129.54 93.98) (width 0.25) (layer F.Cu) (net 13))
 (segment (start 127 76.2) (end 127 78.74) (width 0.25) (layer F.Cu) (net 13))
 (segment (start 129.54 78.74) (end 129.54 76.2) (width 0.3048) (layer F.Cu) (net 13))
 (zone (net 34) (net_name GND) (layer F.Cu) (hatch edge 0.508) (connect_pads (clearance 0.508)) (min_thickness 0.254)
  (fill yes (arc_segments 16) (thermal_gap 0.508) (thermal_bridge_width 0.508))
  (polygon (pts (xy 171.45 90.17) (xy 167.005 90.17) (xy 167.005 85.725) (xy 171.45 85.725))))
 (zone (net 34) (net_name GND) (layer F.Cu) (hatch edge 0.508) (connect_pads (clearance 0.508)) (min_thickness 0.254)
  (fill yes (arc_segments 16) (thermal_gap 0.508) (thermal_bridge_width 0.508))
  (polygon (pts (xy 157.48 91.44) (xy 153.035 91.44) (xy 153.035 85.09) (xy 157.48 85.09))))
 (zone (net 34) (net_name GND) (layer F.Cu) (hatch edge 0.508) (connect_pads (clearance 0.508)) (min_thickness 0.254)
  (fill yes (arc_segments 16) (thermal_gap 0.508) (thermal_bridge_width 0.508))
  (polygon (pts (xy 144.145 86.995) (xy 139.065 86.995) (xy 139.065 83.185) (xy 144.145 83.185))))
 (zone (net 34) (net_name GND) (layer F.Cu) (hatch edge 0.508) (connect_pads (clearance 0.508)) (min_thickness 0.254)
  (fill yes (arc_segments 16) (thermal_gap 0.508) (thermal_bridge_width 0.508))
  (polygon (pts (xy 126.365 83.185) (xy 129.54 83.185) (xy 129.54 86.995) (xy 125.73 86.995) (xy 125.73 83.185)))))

